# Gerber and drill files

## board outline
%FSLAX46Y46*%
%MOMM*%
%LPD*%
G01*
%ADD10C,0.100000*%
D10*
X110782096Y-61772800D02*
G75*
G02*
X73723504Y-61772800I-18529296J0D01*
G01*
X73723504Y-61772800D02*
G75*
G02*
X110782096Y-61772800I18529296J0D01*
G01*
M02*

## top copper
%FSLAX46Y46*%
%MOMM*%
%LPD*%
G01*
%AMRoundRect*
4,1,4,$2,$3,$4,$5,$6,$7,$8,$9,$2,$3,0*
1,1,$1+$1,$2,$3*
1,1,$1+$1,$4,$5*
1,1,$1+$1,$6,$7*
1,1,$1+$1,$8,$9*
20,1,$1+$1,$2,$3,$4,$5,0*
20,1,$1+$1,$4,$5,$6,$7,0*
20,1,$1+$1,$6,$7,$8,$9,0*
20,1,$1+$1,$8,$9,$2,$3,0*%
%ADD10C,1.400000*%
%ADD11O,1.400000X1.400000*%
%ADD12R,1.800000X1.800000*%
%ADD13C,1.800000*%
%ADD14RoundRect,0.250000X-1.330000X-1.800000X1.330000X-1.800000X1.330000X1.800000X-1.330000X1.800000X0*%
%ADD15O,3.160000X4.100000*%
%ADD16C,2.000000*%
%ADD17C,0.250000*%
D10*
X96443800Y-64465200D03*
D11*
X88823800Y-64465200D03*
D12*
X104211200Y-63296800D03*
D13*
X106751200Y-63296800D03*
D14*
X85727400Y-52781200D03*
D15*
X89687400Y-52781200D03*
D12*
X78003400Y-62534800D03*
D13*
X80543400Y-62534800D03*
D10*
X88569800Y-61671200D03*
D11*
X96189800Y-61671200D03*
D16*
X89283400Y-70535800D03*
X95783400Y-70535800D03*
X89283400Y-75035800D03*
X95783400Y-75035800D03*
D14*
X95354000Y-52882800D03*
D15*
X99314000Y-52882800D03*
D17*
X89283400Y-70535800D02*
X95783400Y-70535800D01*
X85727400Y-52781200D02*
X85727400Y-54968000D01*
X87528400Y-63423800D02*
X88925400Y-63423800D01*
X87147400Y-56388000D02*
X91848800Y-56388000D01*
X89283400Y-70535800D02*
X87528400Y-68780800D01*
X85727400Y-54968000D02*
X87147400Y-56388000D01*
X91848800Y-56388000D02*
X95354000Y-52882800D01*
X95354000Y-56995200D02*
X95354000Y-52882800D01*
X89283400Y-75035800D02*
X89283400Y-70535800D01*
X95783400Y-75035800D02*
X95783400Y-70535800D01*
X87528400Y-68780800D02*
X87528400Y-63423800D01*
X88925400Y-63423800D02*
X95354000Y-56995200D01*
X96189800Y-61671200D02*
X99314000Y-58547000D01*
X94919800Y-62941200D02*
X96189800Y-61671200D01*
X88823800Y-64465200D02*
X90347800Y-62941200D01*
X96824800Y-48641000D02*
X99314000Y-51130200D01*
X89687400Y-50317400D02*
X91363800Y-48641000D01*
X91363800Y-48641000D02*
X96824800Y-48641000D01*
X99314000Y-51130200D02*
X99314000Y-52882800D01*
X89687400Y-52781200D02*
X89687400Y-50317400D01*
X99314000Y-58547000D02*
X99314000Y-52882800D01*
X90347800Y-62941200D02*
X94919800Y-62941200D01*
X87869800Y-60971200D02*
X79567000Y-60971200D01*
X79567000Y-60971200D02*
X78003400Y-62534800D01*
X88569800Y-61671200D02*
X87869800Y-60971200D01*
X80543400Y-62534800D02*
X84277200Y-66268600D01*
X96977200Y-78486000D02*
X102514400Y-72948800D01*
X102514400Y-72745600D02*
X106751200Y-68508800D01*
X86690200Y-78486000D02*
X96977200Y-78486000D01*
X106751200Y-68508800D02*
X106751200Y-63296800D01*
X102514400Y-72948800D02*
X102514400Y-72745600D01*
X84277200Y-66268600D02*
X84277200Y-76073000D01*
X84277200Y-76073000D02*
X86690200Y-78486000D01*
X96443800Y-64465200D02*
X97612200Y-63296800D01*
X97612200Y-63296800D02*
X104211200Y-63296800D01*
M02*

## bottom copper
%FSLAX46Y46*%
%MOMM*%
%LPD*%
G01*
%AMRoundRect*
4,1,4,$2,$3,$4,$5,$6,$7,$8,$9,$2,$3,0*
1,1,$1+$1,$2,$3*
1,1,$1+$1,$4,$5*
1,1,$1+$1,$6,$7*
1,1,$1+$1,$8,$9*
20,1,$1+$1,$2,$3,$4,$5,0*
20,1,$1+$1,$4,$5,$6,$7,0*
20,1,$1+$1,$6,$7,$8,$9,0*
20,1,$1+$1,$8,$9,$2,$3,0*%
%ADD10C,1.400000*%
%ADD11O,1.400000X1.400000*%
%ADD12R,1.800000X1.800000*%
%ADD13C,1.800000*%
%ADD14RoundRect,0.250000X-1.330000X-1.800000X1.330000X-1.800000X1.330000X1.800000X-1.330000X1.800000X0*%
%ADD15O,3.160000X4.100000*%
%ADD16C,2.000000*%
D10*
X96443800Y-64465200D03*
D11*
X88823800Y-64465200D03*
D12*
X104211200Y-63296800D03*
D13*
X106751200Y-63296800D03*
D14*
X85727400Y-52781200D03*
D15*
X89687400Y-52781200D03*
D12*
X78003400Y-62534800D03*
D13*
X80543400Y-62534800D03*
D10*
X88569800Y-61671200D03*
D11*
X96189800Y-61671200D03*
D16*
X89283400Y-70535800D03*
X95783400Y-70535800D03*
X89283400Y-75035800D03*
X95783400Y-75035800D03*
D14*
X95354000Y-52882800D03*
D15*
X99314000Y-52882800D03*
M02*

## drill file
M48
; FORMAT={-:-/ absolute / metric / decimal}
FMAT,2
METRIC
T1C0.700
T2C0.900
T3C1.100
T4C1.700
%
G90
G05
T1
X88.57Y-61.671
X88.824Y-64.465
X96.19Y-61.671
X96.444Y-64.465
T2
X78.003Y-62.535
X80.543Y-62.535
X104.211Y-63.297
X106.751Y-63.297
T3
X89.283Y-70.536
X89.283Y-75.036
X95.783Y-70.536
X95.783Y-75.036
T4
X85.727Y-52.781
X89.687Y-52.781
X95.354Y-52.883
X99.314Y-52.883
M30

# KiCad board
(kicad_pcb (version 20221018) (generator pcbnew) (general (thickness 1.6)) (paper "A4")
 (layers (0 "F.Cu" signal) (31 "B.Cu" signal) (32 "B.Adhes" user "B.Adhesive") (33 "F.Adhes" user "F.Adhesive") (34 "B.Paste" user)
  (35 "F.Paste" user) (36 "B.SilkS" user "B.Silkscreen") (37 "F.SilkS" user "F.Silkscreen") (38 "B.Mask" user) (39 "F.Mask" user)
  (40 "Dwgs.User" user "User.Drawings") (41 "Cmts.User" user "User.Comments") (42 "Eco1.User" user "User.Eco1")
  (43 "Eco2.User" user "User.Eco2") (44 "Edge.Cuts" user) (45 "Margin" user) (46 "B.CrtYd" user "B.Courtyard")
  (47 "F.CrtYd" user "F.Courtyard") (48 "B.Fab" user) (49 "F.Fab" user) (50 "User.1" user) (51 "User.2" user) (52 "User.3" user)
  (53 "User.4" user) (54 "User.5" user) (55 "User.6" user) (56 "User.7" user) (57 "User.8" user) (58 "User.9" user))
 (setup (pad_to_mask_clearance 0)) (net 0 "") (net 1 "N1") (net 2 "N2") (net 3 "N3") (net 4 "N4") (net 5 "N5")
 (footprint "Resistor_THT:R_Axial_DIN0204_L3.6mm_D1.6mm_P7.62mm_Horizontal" (layer "F.Cu") (at 96.4438 64.4652 180)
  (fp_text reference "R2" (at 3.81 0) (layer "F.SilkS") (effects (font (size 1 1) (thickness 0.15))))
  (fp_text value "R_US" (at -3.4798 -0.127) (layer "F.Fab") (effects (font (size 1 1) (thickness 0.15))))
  (pad "1" thru_hole circle (at 0 0 180) (size 1.4 1.4) (drill 0.7) (layers "*.Cu" "*.Mask") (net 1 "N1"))
  (pad "2" thru_hole oval (at 7.62 0 180) (size 1.4 1.4) (drill 0.7) (layers "*.Cu" "*.Mask") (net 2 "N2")))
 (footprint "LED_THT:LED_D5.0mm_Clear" (layer "F.Cu") (at 104.2112 63.2968)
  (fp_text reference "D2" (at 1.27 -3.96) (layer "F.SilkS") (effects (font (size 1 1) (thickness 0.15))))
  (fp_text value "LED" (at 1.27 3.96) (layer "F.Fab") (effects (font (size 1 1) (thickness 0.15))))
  (pad "1" thru_hole rect (at 0 0) (size 1.8 1.8) (drill 0.9) (layers "*.Cu" "*.Mask") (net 1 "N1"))
  (pad "2" thru_hole circle (at 2.54 0) (size 1.8 1.8) (drill 0.9) (layers "*.Cu" "*.Mask") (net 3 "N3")))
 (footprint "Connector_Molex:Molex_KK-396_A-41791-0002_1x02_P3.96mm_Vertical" (layer "F.Cu") (at 85.7274 52.7812)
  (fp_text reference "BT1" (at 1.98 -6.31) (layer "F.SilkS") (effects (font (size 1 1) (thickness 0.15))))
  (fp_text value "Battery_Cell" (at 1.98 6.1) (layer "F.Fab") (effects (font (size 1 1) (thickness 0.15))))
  (pad "1" thru_hole roundrect (at 0 0) (size 3.16 4.1) (drill 1.7) (layers "*.Cu" "*.Mask") (roundrect_rratio 0.079114) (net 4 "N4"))
  (pad "2" thru_hole oval (at 3.96 0) (size 3.16 4.1) (drill 1.7) (layers "*.Cu" "*.Mask") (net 2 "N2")))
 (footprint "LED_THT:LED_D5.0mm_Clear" (layer "F.Cu") (at 78.0034 62.5348)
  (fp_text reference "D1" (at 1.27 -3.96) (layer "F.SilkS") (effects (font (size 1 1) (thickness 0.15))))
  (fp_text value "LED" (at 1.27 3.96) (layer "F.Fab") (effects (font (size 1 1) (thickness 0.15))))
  (pad "1" thru_hole rect (at 0 0) (size 1.8 1.8) (drill 0.9) (layers "*.Cu" "*.Mask") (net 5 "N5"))
  (pad "2" thru_hole circle (at 2.54 0) (size 1.8 1.8) (drill 0.9) (layers "*.Cu" "*.Mask") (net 3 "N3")))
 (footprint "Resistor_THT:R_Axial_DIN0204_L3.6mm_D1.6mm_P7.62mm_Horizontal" (layer "F.Cu") (at 88.5698 61.6712)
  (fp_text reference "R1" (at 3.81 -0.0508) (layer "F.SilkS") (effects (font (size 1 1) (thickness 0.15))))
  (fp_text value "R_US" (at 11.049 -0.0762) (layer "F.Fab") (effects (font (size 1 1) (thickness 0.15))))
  (pad "1" thru_hole circle (at 0 0) (size 1.4 1.4) (drill 0.7) (layers "*.Cu" "*.Mask") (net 5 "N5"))
  (pad "2" thru_hole oval (at 7.62 0) (size 1.4 1.4) (drill 0.7) (layers "*.Cu" "*.Mask") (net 2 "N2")))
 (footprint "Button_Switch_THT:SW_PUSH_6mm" (layer "F.Cu") (at 89.2834 70.5358)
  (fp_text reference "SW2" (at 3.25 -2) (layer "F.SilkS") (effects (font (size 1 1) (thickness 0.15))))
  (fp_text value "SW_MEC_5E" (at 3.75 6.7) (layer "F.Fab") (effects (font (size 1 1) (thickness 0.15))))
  (pad "1" thru_hole circle (at 0 0 90) (size 2 2) (drill 1.1) (layers "*.Cu" "*.Mask") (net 4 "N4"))
  (pad "1" thru_hole circle (at 6.5 0 90) (size 2 2) (drill 1.1) (layers "*.Cu" "*.Mask") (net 4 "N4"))
  (pad "2" thru_hole circle (at 0 4.5 90) (size 2 2) (drill 1.1) (layers "*.Cu" "*.Mask") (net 4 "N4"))
  (pad "2" thru_hole circle (at 6.5 4.5 90) (size 2 2) (drill 1.1) (layers "*.Cu" "*.Mask") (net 4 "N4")))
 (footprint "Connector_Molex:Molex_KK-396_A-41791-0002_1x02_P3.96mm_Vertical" (layer "F.Cu") (at 95.354 52.8828)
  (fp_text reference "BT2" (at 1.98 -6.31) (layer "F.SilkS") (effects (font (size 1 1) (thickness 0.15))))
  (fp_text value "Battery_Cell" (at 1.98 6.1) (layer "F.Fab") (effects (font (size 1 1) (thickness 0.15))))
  (pad "1" thru_hole roundrect (at 0 0) (size 3.16 4.1) (drill 1.7) (layers "*.Cu" "*.Mask") (roundrect_rratio 0.079114) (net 4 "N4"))
  (pad "2" thru_hole oval (at 3.96 0) (size 3.16 4.1) (drill 1.7) (layers "*.Cu" "*.Mask") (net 2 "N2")))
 (gr_circle (center 92.2528 61.7728) (end 103.9114 76.1746) (stroke (width 0.1) (type default)) (fill none) (layer "Edge.Cuts"))
 (segment (start 89.2834 70.5358) (end 95.7834 70.5358) (width 0.25) (layer "F.Cu") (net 4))
 (segment (start 85.7274 52.7812) (end 85.7274 54.968) (width 0.25) (layer "F.Cu") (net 4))
 (segment (start 87.5284 63.4238) (end 88.9254 63.4238) (width 0.25) (layer "F.Cu") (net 4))
 (segment (start 87.1474 56.388) (end 91.8488 56.388) (width 0.25) (layer "F.Cu") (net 4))
 (segment (start 89.2834 70.5358) (end 87.5284 68.7808) (width 0.25) (layer "F.Cu") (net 4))
 (segment (start 85.7274 54.968) (end 87.1474 56.388) (width 0.25) (layer "F.Cu") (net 4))
 (segment (start 91.8488 56.388) (end 95.354 52.8828) (width 0.25) (layer "F.Cu") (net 4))
 (segment (start 95.354 56.9952) (end 95.354 52.8828) (width 0.25) (layer "F.Cu") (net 4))
 (segment (start 89.2834 75.0358) (end 89.2834 70.5358) (width 0.25) (layer "F.Cu") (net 4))
 (segment (start 95.7834 75.0358) (end 95.7834 70.5358) (width 0.25) (layer "F.Cu") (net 4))
 (segment (start 87.5284 68.7808) (end 87.5284 63.4238) (width 0.25) (layer "F.Cu") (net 4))
 (segment (start 88.9254 63.4238) (end 95.354 56.9952) (width 0.25) (layer "F.Cu") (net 4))
 (segment (start 96.1898 61.6712) (end 99.314 58.547) (width 0.25) (layer "F.Cu") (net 2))
 (segment (start 94.9198 62.9412) (end 96.1898 61.6712) (width 0.25) (layer "F.Cu") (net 2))
 (segment (start 88.8238 64.4652) (end 90.3478 62.9412) (width 0.25) (layer "F.Cu") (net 2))
 (segment (start 96.8248 48.641) (end 99.314 51.1302) (width 0.25) (layer "F.Cu") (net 2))
 (segment (start 89.6874 50.3174) (end 91.3638 48.641) (width 0.25) (layer "F.Cu") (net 2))
 (segment (start 91.3638 48.641) (end 96.8248 48.641) (width 0.25) (layer "F.Cu") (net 2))
 (segment (start 99.314 51.1302) (end 99.314 52.8828) (width 0.25) (layer "F.Cu") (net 2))
 (segment (start 89.6874 52.7812) (end 89.6874 50.3174) (width 0.25) (layer "F.Cu") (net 2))
 (segment (start 99.314 58.547) (end 99.314 52.8828) (width 0.25) (layer "F.Cu") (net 2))
 (segment (start 90.3478 62.9412) (end 94.9198 62.9412) (width 0.25) (layer "F.Cu") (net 2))
 (segment (start 87.8698 60.9712) (end 79.567 60.9712) (width 0.25) (layer "F.Cu") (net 5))
 (segment (start 79.567 60.9712) (end 78.0034 62.5348) (width 0.25) (layer "F.Cu") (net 5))
 (segment (start 88.5698 61.6712) (end 87.8698 60.9712) (width 0.25) (layer "F.Cu") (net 5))
 (segment (start 80.5434 62.5348) (end 84.2772 66.2686) (width 0.25) (layer "F.Cu") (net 3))
 (segment (start 96.9772 78.486) (end 102.5144 72.9488) (width 0.25) (layer "F.Cu") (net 3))
 (segment (start 102.5144 72.7456) (end 106.7512 68.5088) (width 0.25) (layer "F.Cu") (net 3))
 (segment (start 86.6902 78.486) (end 96.9772 78.486) (width 0.25) (layer "F.Cu") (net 3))
 (segment (start 106.7512 68.5088) (end 106.7512 63.2968) (width 0.25) (layer "F.Cu") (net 3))
 (segment (start 102.5144 72.9488) (end 102.5144 72.7456) (width 0.25) (layer "F.Cu") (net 3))
 (segment (start 84.2772 66.2686) (end 84.2772 76.073) (width 0.25) (layer "F.Cu") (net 3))
 (segment (start 84.2772 76.073) (end 86.6902 78.486) (width 0.25) (layer "F.Cu") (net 3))
 (segment (start 96.4438 64.4652) (end 97.6122 63.2968) (width 0.25) (layer "F.Cu") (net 1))
 (segment (start 97.6122 63.2968) (end 104.2112 63.2968) (width 0.25) (layer "F.Cu") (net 1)))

